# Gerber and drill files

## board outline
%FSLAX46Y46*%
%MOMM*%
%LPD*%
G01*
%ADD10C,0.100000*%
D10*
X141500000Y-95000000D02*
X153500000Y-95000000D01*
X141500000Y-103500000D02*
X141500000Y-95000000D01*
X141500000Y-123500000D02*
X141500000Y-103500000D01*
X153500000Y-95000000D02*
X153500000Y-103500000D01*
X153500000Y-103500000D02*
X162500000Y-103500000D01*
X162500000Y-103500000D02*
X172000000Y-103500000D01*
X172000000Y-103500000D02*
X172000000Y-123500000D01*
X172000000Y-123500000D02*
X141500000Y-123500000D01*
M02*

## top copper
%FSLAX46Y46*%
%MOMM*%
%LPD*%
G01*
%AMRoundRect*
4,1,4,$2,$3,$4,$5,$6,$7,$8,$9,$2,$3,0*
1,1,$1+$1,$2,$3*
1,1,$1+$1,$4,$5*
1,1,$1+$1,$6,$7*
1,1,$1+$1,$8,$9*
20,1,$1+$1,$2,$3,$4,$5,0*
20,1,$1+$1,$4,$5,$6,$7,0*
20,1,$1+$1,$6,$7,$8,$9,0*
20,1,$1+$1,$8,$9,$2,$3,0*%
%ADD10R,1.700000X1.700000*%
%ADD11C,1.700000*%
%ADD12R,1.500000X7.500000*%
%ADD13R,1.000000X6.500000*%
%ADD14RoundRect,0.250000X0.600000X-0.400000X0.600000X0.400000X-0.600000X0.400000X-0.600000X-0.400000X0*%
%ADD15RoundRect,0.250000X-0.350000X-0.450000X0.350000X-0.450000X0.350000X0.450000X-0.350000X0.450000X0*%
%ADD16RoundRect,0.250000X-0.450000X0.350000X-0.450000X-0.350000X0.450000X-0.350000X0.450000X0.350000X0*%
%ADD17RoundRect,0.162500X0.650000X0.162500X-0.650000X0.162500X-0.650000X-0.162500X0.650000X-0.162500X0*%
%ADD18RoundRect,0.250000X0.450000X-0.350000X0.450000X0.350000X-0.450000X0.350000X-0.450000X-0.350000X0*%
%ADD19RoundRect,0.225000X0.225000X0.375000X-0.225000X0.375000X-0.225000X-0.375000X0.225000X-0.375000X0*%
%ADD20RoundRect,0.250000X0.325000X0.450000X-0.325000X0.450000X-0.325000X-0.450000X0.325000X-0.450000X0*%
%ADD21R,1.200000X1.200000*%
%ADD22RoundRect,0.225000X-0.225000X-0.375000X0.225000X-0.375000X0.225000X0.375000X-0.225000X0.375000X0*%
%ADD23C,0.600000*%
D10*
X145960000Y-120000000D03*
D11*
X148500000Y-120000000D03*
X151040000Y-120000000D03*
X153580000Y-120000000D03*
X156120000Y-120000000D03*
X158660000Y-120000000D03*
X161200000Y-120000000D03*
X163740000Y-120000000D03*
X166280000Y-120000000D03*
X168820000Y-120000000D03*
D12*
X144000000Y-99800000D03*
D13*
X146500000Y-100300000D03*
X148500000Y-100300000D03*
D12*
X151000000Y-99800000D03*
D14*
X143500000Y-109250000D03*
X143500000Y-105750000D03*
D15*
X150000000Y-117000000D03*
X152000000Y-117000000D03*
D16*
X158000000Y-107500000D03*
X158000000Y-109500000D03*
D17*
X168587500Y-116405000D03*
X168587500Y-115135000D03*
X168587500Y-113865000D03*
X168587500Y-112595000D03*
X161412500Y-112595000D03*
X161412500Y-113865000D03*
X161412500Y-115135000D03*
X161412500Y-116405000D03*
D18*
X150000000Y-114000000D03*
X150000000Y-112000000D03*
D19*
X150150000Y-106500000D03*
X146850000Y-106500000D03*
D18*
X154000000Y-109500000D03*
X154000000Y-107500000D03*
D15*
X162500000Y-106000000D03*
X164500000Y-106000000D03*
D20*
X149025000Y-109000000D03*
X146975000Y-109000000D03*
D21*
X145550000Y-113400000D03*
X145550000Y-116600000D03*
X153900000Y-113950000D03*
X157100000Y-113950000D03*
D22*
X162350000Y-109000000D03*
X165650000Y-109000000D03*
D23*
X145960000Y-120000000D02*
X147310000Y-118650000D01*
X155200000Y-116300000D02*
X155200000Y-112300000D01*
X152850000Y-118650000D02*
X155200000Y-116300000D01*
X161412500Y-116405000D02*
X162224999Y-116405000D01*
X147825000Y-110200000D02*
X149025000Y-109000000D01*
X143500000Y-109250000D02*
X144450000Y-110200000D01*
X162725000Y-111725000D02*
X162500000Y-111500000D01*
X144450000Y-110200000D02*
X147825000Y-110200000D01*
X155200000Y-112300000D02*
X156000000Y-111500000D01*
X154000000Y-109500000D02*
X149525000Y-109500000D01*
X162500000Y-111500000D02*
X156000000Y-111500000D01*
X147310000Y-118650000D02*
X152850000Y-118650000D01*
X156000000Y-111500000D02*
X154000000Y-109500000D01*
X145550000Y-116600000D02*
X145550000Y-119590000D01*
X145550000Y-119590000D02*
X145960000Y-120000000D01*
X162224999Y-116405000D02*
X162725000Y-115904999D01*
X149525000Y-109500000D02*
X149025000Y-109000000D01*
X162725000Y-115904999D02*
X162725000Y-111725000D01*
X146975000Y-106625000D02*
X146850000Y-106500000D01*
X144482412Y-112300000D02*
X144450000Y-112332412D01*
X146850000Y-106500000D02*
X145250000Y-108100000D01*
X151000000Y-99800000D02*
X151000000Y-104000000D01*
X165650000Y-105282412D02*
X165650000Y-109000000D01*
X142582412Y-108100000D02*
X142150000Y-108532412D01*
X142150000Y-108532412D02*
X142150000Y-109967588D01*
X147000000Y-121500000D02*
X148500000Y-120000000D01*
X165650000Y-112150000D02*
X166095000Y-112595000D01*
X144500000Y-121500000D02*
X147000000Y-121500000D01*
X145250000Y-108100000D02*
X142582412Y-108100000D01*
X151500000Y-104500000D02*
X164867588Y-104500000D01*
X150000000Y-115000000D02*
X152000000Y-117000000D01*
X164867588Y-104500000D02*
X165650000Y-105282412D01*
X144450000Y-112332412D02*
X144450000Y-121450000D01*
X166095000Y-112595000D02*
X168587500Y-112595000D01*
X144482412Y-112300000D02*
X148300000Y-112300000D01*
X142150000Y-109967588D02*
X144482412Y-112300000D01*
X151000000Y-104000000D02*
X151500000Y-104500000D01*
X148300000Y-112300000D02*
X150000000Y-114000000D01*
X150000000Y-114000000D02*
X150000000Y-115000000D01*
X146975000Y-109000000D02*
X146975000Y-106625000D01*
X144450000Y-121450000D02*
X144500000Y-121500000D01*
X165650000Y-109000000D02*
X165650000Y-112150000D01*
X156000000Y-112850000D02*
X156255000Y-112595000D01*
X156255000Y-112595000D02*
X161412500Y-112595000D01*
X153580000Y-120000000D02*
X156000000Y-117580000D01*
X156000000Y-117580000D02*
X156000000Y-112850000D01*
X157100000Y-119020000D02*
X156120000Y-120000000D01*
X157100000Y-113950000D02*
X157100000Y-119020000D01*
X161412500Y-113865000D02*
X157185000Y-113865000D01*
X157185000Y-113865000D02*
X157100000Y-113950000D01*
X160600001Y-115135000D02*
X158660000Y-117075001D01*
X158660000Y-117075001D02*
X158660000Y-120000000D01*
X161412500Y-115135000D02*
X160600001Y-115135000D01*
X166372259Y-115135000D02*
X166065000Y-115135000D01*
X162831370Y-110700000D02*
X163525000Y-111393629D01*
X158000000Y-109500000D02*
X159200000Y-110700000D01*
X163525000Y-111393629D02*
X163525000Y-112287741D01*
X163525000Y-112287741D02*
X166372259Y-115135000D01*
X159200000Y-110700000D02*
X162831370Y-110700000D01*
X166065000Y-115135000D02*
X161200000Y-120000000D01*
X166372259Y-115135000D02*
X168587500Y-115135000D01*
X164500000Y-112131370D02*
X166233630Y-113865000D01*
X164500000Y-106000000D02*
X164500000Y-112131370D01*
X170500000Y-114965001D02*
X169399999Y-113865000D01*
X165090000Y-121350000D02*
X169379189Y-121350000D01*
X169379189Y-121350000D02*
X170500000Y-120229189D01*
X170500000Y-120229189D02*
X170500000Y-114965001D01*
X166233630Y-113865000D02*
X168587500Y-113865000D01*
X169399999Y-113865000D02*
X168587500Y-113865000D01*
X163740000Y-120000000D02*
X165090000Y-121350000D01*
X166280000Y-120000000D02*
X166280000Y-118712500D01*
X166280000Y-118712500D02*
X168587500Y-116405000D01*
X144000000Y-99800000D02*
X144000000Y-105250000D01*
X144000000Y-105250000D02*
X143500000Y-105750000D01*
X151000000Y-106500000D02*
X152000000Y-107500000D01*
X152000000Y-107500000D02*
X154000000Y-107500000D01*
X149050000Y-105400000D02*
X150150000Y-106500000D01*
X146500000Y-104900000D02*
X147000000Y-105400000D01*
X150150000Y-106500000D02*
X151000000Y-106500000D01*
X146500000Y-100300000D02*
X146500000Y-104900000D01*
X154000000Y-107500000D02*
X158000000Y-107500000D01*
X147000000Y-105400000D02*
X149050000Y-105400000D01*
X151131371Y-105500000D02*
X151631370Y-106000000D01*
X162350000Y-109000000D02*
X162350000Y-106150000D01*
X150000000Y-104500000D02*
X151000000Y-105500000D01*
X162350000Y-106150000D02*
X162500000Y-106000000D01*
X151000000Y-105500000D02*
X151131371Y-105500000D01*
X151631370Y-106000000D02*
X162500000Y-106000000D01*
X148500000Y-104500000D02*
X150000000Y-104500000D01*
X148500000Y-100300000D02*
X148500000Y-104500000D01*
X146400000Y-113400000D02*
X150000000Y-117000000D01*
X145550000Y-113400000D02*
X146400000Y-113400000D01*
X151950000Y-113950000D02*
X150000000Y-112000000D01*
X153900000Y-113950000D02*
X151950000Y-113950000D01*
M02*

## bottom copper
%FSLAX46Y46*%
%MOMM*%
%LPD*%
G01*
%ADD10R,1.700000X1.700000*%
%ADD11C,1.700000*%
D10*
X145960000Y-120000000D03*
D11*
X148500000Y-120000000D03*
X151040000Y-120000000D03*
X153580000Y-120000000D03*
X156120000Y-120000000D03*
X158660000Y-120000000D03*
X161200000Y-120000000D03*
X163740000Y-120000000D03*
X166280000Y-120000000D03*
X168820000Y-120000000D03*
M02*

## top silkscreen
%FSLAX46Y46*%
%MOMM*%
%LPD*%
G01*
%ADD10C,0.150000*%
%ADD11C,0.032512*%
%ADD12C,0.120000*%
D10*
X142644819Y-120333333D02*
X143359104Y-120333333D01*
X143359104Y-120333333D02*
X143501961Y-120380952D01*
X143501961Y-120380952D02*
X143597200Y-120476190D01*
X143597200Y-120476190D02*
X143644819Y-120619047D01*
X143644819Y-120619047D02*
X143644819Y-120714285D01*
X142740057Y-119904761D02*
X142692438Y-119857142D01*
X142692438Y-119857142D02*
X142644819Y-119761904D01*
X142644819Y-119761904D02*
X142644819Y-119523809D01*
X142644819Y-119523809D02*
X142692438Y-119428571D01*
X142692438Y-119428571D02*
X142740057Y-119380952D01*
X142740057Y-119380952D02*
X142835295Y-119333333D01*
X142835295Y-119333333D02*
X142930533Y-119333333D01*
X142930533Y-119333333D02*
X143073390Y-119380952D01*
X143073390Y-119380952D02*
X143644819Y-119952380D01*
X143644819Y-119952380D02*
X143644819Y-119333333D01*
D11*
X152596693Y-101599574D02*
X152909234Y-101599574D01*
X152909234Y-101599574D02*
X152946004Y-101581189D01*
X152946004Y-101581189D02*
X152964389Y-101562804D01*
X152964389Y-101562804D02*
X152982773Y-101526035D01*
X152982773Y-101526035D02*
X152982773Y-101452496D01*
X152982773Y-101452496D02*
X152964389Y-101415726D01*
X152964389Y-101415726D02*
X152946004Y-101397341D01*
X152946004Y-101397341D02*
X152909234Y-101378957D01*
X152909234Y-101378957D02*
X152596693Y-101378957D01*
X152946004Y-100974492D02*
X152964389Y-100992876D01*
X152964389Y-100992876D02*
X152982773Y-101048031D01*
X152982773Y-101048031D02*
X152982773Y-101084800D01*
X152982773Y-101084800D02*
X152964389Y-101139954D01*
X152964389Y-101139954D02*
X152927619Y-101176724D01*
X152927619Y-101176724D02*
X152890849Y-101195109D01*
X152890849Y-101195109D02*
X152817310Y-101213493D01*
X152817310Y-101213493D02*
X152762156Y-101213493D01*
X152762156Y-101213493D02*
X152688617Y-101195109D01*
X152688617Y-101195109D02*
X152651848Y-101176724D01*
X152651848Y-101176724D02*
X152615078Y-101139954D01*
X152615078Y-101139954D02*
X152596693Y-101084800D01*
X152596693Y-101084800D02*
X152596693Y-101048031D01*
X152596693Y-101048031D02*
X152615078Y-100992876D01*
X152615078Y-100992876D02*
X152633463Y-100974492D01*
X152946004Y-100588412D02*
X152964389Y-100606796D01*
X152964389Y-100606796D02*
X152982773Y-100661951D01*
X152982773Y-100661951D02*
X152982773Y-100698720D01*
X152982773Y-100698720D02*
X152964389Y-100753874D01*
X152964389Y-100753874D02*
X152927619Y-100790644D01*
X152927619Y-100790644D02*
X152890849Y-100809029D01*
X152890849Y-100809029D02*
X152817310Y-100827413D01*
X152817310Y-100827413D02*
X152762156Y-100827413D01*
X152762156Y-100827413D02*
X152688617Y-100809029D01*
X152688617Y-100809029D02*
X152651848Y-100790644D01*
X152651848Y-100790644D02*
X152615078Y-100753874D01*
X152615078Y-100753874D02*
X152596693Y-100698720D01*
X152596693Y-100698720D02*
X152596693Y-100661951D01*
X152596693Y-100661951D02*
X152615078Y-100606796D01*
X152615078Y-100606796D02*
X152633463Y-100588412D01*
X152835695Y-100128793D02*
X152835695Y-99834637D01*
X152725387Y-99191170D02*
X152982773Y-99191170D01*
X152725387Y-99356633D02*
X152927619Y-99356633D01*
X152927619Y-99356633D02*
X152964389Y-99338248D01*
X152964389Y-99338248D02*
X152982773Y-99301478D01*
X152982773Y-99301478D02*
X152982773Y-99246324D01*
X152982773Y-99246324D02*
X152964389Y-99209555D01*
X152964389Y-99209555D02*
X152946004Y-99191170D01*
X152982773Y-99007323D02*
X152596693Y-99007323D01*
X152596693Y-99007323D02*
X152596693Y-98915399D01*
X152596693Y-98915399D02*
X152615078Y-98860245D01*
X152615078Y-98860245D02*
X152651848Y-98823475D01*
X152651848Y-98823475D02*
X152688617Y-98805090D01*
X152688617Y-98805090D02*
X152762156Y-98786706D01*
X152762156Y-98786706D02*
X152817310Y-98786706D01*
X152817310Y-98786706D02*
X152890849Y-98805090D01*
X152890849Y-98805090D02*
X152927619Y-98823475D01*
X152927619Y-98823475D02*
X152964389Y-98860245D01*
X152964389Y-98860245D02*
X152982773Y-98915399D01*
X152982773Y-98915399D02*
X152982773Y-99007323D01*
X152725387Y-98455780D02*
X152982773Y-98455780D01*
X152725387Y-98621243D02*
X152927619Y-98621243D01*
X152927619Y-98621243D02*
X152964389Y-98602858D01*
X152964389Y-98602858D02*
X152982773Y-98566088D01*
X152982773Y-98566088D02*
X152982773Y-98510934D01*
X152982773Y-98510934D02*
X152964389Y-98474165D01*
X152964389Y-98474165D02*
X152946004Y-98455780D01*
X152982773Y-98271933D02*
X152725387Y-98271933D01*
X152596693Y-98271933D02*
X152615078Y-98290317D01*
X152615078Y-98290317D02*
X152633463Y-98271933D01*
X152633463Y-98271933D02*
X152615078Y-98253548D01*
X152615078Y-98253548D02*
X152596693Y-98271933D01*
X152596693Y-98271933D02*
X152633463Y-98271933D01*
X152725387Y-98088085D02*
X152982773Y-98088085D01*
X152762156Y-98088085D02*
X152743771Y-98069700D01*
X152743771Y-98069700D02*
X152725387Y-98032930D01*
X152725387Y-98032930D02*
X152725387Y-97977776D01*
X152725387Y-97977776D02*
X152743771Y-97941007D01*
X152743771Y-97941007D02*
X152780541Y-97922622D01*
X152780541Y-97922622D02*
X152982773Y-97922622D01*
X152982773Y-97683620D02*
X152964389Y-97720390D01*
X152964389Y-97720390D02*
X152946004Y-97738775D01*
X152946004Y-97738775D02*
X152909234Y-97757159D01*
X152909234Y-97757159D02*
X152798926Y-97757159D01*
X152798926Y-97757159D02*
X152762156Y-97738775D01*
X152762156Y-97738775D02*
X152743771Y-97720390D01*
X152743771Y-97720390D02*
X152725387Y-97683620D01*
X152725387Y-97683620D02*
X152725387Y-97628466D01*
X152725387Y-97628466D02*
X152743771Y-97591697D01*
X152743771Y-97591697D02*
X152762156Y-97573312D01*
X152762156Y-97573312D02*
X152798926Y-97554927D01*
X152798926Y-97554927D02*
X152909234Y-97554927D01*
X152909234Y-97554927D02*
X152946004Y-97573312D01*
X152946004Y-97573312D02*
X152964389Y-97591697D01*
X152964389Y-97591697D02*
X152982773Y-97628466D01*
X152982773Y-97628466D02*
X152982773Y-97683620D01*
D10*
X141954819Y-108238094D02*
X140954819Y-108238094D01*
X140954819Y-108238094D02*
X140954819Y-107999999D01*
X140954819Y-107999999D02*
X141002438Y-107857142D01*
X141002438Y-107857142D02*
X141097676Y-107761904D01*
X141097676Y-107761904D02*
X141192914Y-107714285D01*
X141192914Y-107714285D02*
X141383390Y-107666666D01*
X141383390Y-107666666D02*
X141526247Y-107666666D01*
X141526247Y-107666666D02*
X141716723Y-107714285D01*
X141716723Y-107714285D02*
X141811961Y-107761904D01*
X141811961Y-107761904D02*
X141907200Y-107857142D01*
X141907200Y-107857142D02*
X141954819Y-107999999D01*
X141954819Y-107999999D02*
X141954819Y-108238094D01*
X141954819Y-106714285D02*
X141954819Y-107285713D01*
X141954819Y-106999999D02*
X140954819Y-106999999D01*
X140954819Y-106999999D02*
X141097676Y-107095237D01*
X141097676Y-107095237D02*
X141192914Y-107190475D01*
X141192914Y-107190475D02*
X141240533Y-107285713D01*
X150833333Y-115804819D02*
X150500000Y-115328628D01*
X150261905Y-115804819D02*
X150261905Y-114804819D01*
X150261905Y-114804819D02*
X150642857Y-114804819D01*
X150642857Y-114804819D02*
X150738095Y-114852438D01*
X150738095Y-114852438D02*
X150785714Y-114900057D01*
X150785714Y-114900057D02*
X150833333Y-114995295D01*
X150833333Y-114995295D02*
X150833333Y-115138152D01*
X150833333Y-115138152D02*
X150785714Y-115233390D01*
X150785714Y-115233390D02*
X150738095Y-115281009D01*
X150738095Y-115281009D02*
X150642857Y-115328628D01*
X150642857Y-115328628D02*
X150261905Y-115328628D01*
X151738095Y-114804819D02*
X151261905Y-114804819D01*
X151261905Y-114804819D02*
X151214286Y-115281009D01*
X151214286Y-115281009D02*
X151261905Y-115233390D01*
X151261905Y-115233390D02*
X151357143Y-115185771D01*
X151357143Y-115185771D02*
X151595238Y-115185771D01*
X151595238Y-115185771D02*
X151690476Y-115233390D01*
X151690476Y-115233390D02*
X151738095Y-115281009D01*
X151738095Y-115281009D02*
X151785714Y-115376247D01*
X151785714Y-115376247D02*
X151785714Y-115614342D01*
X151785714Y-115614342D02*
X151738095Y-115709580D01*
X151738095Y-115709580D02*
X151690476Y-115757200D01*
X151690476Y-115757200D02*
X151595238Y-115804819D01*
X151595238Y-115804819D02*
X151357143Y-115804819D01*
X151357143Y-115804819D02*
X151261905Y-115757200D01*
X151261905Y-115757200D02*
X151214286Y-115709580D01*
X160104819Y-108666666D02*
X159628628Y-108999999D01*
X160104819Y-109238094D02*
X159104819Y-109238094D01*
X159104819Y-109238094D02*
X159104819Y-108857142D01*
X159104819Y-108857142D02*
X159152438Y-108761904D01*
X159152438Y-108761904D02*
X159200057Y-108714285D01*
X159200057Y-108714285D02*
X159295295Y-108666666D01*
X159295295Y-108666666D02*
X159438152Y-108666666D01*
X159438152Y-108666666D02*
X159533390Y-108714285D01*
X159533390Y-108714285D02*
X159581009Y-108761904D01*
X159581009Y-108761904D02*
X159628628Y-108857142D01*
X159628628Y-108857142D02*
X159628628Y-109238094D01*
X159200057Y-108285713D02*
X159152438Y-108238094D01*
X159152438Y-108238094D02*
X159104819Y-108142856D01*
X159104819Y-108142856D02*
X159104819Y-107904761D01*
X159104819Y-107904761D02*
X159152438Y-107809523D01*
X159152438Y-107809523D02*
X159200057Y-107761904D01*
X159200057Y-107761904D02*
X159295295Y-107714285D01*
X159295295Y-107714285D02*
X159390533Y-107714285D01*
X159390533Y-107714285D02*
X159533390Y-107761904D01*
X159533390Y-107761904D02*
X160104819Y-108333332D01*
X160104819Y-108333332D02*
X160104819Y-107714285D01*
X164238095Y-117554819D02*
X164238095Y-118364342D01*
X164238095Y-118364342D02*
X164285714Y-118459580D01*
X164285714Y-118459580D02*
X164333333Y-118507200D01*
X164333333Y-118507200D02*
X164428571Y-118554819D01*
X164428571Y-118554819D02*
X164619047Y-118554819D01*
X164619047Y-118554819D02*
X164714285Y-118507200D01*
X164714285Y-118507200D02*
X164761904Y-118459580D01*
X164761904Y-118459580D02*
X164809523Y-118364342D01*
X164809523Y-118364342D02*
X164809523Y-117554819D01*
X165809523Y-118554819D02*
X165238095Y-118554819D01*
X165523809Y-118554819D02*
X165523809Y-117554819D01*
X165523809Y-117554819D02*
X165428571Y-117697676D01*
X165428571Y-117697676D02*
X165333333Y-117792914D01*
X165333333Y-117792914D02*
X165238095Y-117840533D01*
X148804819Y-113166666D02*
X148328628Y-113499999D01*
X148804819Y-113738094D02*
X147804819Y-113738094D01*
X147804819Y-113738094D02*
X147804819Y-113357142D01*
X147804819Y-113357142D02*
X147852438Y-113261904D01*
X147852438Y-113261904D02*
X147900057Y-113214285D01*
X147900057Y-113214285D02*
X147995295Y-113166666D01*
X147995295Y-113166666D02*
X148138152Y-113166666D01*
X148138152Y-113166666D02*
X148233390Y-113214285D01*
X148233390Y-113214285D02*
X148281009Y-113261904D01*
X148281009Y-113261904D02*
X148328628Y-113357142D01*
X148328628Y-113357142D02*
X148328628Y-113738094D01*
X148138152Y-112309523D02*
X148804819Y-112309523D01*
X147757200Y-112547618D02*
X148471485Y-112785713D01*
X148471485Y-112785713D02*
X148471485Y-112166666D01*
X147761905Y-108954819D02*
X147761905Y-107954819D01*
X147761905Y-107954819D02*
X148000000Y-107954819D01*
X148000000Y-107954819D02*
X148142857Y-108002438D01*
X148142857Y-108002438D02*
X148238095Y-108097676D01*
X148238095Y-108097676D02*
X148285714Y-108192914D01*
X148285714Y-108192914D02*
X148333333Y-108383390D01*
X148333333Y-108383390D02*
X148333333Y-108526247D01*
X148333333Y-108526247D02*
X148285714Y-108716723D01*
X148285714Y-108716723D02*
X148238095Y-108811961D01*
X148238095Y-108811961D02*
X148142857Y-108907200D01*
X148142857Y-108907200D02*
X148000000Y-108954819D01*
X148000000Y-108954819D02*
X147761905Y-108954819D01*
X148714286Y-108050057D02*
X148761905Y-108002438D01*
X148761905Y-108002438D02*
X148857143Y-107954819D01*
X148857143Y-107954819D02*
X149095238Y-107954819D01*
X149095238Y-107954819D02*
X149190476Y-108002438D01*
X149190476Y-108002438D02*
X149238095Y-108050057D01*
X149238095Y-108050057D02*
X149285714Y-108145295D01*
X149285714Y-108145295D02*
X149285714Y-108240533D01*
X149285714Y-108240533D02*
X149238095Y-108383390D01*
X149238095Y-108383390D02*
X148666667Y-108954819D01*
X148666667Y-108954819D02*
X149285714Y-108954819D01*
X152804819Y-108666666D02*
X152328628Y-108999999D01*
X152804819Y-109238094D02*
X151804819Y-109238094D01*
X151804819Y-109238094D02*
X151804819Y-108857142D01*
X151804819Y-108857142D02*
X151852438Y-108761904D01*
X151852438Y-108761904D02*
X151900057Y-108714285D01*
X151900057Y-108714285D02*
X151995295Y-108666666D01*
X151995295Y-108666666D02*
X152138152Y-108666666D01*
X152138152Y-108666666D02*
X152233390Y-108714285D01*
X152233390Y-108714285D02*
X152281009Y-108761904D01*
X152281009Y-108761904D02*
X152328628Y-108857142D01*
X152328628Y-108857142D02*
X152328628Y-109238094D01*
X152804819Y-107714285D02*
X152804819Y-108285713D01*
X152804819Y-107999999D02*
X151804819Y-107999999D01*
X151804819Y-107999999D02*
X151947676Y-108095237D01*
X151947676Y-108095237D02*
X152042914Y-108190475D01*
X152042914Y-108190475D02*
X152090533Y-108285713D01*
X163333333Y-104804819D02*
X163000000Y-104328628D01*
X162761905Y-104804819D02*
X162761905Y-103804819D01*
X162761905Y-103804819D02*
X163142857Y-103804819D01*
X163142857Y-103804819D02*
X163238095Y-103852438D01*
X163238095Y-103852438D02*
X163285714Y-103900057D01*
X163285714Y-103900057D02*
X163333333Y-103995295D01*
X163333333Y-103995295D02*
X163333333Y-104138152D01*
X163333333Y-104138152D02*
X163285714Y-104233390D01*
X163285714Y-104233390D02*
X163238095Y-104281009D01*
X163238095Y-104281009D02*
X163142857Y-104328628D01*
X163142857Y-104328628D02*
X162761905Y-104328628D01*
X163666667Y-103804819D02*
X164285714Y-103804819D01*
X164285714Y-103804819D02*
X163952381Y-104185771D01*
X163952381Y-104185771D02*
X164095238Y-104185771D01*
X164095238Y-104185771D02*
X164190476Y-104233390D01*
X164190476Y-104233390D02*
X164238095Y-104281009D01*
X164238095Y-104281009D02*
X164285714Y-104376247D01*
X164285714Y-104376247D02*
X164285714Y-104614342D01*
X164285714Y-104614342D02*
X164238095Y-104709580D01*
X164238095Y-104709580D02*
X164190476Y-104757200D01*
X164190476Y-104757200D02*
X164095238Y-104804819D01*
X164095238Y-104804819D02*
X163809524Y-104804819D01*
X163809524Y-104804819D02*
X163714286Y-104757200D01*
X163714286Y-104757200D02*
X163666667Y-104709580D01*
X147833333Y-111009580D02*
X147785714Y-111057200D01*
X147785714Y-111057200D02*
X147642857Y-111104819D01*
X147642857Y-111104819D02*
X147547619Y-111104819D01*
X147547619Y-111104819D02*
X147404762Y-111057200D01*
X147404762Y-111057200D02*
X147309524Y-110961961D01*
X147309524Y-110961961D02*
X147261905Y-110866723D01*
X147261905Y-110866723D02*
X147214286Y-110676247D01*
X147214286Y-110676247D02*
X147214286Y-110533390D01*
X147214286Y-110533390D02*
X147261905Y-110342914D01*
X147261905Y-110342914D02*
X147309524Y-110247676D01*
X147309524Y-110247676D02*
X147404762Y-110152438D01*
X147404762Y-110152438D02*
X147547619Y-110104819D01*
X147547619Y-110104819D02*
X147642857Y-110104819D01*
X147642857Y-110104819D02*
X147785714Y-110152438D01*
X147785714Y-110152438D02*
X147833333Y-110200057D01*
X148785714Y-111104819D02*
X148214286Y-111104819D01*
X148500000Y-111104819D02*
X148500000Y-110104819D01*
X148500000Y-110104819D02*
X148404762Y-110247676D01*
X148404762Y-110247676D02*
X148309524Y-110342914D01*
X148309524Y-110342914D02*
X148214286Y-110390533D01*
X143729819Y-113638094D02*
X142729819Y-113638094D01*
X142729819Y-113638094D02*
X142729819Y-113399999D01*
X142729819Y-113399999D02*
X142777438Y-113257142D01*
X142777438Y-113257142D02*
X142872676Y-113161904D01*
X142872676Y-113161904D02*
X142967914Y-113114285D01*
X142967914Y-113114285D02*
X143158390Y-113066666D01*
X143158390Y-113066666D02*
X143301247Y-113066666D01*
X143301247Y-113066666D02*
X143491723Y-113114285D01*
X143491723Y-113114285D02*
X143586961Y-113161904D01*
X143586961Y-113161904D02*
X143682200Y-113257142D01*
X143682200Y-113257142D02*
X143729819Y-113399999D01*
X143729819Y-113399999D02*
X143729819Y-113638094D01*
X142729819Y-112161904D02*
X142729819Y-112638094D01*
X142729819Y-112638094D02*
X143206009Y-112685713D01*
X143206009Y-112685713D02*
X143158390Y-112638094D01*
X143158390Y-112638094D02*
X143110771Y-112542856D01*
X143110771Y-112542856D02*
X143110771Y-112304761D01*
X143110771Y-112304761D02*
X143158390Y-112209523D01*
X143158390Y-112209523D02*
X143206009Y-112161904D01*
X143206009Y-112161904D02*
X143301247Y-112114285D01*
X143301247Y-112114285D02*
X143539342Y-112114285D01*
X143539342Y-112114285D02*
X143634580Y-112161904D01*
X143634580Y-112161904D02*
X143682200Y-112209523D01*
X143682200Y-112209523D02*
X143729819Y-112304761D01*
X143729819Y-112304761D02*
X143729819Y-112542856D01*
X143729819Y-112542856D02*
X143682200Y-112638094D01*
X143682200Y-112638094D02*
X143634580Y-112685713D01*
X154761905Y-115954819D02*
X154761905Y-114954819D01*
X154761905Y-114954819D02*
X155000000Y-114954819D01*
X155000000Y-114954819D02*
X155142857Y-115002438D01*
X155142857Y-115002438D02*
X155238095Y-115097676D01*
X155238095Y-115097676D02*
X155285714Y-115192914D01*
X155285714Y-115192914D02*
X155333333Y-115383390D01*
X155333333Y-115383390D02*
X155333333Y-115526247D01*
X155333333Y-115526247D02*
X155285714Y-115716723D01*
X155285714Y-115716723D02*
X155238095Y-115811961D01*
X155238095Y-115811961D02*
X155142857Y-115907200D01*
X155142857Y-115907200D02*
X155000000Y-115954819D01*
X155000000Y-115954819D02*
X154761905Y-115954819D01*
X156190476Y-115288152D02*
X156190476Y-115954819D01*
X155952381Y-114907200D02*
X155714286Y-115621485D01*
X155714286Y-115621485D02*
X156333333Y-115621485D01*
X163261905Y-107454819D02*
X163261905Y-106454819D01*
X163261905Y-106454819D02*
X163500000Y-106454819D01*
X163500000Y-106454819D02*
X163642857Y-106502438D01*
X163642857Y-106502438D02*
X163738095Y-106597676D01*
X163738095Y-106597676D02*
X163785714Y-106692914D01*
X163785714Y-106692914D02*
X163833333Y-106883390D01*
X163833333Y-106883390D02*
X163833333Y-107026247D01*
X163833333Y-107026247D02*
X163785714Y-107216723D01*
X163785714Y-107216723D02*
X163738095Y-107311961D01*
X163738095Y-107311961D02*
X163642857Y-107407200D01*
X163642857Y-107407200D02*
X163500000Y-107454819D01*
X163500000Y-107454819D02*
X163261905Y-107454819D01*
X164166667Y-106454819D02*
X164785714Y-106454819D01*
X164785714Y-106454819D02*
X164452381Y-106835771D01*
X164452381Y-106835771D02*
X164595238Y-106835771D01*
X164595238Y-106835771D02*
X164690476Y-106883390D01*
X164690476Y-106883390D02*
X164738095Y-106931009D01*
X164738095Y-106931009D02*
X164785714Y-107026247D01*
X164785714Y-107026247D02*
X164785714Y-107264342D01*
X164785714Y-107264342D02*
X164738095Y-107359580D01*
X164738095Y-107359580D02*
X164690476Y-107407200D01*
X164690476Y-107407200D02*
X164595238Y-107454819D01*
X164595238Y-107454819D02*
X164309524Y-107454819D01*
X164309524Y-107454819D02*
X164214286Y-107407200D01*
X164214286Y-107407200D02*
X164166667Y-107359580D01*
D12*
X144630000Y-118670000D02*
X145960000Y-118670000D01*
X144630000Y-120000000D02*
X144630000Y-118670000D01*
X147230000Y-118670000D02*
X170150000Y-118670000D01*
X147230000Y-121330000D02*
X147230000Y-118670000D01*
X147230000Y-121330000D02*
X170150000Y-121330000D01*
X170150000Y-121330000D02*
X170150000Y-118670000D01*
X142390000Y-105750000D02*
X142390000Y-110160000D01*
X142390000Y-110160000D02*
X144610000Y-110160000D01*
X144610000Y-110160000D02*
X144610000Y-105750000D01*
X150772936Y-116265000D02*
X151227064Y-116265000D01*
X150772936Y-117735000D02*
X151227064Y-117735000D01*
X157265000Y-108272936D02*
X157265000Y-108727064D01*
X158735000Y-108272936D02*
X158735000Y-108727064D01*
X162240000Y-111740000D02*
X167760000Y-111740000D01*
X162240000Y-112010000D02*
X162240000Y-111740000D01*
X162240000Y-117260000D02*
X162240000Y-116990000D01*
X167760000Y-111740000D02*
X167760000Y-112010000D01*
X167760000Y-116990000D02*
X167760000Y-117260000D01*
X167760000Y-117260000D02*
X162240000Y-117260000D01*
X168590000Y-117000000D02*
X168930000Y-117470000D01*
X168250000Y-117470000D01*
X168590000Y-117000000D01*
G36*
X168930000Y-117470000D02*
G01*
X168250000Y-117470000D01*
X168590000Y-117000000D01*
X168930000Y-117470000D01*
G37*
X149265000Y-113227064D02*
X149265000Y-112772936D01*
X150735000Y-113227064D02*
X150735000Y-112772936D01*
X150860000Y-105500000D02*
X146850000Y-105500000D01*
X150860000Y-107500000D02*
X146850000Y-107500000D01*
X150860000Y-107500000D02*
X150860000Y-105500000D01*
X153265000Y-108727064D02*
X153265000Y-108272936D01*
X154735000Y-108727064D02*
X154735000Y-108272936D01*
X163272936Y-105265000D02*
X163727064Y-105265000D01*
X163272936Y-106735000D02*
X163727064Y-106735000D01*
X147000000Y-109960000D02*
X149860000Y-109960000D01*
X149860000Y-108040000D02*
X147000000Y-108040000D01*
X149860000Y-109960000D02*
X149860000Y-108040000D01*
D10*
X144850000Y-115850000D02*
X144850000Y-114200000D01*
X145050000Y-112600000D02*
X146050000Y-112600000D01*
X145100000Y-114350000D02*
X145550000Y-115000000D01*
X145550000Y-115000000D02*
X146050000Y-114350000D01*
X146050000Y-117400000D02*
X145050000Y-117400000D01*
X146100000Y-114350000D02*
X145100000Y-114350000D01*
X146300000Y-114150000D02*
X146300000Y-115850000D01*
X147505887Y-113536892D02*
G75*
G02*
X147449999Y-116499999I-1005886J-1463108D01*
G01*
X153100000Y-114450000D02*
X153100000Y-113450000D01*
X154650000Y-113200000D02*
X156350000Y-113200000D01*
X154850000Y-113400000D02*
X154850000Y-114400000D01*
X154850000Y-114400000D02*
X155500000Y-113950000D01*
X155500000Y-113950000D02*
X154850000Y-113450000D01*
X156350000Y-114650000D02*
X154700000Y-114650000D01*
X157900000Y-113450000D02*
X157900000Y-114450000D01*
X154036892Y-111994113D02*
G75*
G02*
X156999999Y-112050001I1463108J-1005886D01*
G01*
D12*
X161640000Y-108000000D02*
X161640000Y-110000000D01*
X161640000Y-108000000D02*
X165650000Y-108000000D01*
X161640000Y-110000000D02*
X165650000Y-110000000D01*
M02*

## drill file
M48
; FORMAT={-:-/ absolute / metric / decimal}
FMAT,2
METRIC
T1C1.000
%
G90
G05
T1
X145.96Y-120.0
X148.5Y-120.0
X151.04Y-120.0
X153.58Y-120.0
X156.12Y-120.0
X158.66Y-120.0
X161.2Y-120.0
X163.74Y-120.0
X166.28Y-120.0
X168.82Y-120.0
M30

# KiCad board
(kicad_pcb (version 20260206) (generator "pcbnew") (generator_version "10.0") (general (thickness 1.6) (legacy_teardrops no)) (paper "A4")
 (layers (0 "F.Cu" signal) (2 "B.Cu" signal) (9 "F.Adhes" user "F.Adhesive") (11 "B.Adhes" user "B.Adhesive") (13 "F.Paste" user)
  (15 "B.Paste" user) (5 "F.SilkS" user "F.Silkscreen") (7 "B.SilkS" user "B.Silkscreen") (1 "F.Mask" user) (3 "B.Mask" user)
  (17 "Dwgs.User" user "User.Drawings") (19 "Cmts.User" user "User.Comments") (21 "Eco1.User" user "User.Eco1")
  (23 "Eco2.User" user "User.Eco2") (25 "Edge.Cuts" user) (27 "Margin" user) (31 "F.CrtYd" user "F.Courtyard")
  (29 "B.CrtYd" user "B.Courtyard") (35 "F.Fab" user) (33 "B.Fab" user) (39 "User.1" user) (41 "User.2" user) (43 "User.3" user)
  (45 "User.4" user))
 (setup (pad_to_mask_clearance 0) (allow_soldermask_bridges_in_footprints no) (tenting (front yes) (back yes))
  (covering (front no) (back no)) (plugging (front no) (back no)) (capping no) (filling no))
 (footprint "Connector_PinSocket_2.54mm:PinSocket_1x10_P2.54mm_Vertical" (layer "F.Cu") (at 145.96 120 90)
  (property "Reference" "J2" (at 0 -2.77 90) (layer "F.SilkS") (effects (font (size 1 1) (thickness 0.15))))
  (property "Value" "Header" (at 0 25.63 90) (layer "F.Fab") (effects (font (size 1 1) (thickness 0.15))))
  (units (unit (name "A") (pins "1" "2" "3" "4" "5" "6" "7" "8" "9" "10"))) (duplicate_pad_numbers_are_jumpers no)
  (fp_line (start 1.33 -1.33) (end 1.33 0) (stroke (width 0.12) (type solid)) (layer "F.SilkS"))
  (fp_line (start 0 -1.33) (end 1.33 -1.33) (stroke (width 0.12) (type solid)) (layer "F.SilkS"))
  (fp_line (start 1.33 1.27) (end 1.33 24.19) (stroke (width 0.12) (type solid)) (layer "F.SilkS"))
  (fp_line (start -1.33 1.27) (end 1.33 1.27) (stroke (width 0.12) (type solid)) (layer "F.SilkS"))
  (fp_line (start -1.33 1.27) (end -1.33 24.19) (stroke (width 0.12) (type solid)) (layer "F.SilkS"))
  (fp_line (start -1.33 24.19) (end 1.33 24.19) (stroke (width 0.12) (type solid)) (layer "F.SilkS"))
  (pad "1" thru_hole rect (at 0 0 90) (size 1.7 1.7) (drill 1) (layers "*.Cu" "*.Mask") (remove_unused_layers no) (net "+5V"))
  (pad "2" thru_hole circle (at 0 2.54 90) (size 1.7 1.7) (drill 1) (layers "*.Cu" "*.Mask") (remove_unused_layers no) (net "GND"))
  (pad "3" thru_hole circle (at 0 5.08 90) (size 1.7 1.7) (drill 1) (layers "*.Cu" "*.Mask") (remove_unused_layers no)
   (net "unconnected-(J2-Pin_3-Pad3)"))
  (pad "4" thru_hole circle (at 0 7.62 90) (size 1.7 1.7) (drill 1) (layers "*.Cu" "*.Mask") (remove_unused_layers no)
   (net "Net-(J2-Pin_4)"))
  (pad "5" thru_hole circle (at 0 10.16 90) (size 1.7 1.7) (drill 1) (layers "*.Cu" "*.Mask") (remove_unused_layers no) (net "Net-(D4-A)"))
  (pad "6" thru_hole circle (at 0 12.7 90) (size 1.7 1.7) (drill 1) (layers "*.Cu" "*.Mask") (remove_unused_layers no)
   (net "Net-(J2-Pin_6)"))
  (pad "7" thru_hole circle (at 0 15.24 90) (size 1.7 1.7) (drill 1) (layers "*.Cu" "*.Mask") (remove_unused_layers no)
   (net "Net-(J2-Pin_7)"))
  (pad "8" thru_hole circle (at 0 17.78 90) (size 1.7 1.7) (drill 1) (layers "*.Cu" "*.Mask") (remove_unused_layers no)
   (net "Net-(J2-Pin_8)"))
  (pad "9" thru_hole circle (at 0 20.32 90) (size 1.7 1.7) (drill 1) (layers "*.Cu" "*.Mask") (remove_unused_layers no)
   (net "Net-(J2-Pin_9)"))
  (pad "10" thru_hole circle (at 0 22.86 90) (size 1.7 1.7) (drill 1) (layers "*.Cu" "*.Mask") (remove_unused_layers no)
   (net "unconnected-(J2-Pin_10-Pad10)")))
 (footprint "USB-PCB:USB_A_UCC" (layer "F.Cu") (at 147.5 100 -90)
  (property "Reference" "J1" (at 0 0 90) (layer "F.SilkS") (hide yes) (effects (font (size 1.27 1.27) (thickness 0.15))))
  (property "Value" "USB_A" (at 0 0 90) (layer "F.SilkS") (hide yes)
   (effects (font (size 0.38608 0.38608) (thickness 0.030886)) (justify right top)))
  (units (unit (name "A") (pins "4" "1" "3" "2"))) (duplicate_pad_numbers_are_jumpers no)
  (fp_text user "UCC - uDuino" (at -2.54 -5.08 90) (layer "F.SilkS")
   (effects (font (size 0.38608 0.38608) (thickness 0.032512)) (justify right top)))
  (pad "1" smd rect (at -0.2 3.5 270) (size 7.5 1.5) (layers "F.Cu" "F.Mask" "F.Paste") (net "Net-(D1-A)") (solder_mask_margin 0.1016))
  (pad "2" smd rect (at 0.3 1 270) (size 6.5 1) (layers "F.Cu" "F.Mask" "F.Paste") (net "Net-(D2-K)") (solder_mask_margin 0.1016))
  (pad "3" smd rect (at 0.3 -1 270) (size 6.5 1) (layers "F.Cu" "F.Mask" "F.Paste") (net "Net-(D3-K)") (solder_mask_margin 0.1016))
  (pad "4" smd rect (at -0.2 -3.5 270) (size 7.5 1.5) (layers "F.Cu" "F.Mask" "F.Paste") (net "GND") (solder_mask_margin 0.1016)))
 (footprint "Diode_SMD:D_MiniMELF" (layer "F.Cu") (at 143.5 107.5 90)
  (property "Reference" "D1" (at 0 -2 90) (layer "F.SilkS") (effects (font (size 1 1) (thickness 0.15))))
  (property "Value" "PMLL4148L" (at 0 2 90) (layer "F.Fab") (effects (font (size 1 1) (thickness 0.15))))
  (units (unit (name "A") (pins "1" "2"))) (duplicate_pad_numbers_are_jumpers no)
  (fp_line (start 1.75 -1.11) (end -2.66 -1.11) (stroke (width 0.12) (type solid)) (layer "F.SilkS"))
  (fp_line (start -2.66 -1.11) (end -2.66 1.11) (stroke (width 0.12) (type solid)) (layer "F.SilkS"))
  (fp_line (start -2.66 1.11) (end 1.75 1.11) (stroke (width 0.12) (type solid)) (layer "F.SilkS"))
  (pad "1" smd roundrect (at -1.75 0 90) (size 1.3 1.7) (layers "F.Cu" "F.Mask" "F.Paste") (roundrect_rratio 0.1923076923) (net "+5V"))
  (pad "2" smd roundrect (at 1.75 0 90) (size 1.3 1.7) (layers "F.Cu" "F.Mask" "F.Paste") (roundrect_rratio 0.1923076923) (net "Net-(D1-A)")))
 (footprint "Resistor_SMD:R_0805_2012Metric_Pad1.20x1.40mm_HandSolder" (layer "F.Cu") (at 151 117)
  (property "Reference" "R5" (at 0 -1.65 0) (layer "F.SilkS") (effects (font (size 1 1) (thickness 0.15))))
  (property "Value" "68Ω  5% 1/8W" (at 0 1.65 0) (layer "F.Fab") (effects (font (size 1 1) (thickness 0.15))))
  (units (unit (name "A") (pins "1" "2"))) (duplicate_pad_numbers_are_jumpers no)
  (fp_line (start -0.227064 -0.735) (end 0.227064 -0.735) (stroke (width 0.12) (type solid)) (layer "F.SilkS"))
  (fp_line (start -0.227064 0.735) (end 0.227064 0.735) (stroke (width 0.12) (type solid)) (layer "F.SilkS"))
  (pad "1" smd roundrect (at -1 0) (size 1.2 1.4) (layers "F.Cu" "F.Mask" "F.Paste") (roundrect_rratio 0.208333) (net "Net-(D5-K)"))
  (pad "2" smd roundrect (at 1 0) (size 1.2 1.4) (layers "F.Cu" "F.Mask" "F.Paste") (roundrect_rratio 0.208333) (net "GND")))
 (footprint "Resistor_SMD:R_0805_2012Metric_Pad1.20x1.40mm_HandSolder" (layer "F.Cu") (at 158 108.5 -90)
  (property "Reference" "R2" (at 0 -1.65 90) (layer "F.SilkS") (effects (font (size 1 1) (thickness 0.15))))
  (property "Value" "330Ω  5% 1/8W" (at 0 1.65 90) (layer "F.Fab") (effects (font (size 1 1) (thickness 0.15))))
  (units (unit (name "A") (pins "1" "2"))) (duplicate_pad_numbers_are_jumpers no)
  (fp_line (start -0.227064 0.735) (end 0.227064 0.735) (stroke (width 0.12) (type solid)) (layer "F.SilkS"))
  (fp_line (start -0.227064 -0.735) (end 0.227064 -0.735) (stroke (width 0.12) (type solid)) (layer "F.SilkS"))
  (pad "1" smd roundrect (at -1 0 270) (size 1.2 1.4) (layers "F.Cu" "F.Mask" "F.Paste") (roundrect_rratio 0.208333) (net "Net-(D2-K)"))
  (pad "2" smd roundrect (at 1 0 270) (size 1.2 1.4) (layers "F.Cu" "F.Mask" "F.Paste") (roundrect_rratio 0.208333) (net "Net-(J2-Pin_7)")))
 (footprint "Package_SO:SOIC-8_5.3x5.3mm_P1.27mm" (layer "F.Cu") (at 165 114.5 180)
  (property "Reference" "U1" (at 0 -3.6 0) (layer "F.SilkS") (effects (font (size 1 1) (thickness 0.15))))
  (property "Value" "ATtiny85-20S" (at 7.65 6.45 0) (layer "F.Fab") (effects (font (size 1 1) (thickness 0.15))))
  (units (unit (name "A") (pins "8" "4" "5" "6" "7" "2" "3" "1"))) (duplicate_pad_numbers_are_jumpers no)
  (fp_line (start 2.76 2.76) (end -2.76 2.76) (stroke (width 0.12) (type solid)) (layer "F.SilkS"))
  (fp_line (start 2.76 2.49) (end 2.76 2.76) (stroke (width 0.12) (type solid)) (layer "F.SilkS"))
  (fp_line (start 2.76 -2.76) (end 2.76 -2.49) (stroke (width 0.12) (type solid)) (layer "F.SilkS"))
  (fp_line (start -2.76 2.76) (end -2.76 2.49) (stroke (width 0.12) (type solid)) (layer "F.SilkS"))
  (fp_line (start -2.76 -2.49) (end -2.76 -2.76) (stroke (width 0.12) (type solid)) (layer "F.SilkS"))
  (fp_line (start -2.76 -2.76) (end 2.76 -2.76) (stroke (width 0.12) (type solid)) (layer "F.SilkS"))
  (fp_poly (pts (xy -3.59 -2.5) (xy -3.93 -2.97) (xy -3.25 -2.97)) (stroke (width 0.12) (type solid)) (fill yes) (layer "F.SilkS"))
  (pad "1" smd roundrect (at -3.5875 -1.905 180) (size 1.625 0.65) (layers "F.Cu" "F.Mask" "F.Paste") (roundrect_rratio 0.25)
   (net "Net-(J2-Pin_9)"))
  (pad "2" smd roundrect (at -3.5875 -0.635 180) (size 1.625 0.65) (layers "F.Cu" "F.Mask" "F.Paste") (roundrect_rratio 0.25)
   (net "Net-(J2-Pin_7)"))
  (pad "3" smd roundrect (at -3.5875 0.635 180) (size 1.625 0.65) (layers "F.Cu" "F.Mask" "F.Paste") (roundrect_rratio 0.25)
   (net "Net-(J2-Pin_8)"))
  (pad "4" smd roundrect (at -3.5875 1.905 180) (size 1.625 0.65) (layers "F.Cu" "F.Mask" "F.Paste") (roundrect_rratio 0.25) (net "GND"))
  (pad "5" smd roundrect (at 3.5875 1.905 180) (size 1.625 0.65) (layers "F.Cu" "F.Mask" "F.Paste") (roundrect_rratio 0.25)
   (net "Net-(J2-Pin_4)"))
  (pad "6" smd roundrect (at 3.5875 0.635 180) (size 1.625 0.65) (layers "F.Cu" "F.Mask" "F.Paste") (roundrect_rratio 0.25)
   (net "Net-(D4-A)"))
  (pad "7" smd roundrect (at 3.5875 -0.635 180) (size 1.625 0.65) (layers "F.Cu" "F.Mask" "F.Paste") (roundrect_rratio 0.25)
   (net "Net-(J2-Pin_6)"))
  (pad "8" smd roundrect (at 3.5875 -1.905 180) (size 1.625 0.65) (layers "F.Cu" "F.Mask" "F.Paste") (roundrect_rratio 0.25) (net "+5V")))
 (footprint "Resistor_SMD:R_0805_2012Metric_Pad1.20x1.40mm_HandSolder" (layer "F.Cu") (at 150 113 90)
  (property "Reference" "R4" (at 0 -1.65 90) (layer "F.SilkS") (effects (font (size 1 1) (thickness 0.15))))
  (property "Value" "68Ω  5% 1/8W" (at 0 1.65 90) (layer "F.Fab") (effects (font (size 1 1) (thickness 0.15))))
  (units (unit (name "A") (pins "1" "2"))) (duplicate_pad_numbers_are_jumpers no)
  (fp_line (start -0.227064 -0.735) (end 0.227064 -0.735) (stroke (width 0.12) (type solid)) (layer "F.SilkS"))
  (fp_line (start -0.227064 0.735) (end 0.227064 0.735) (stroke (width 0.12) (type solid)) (layer "F.SilkS"))
  (pad "1" smd roundrect (at -1 0 90) (size 1.2 1.4) (layers "F.Cu" "F.Mask" "F.Paste") (roundrect_rratio 0.208333) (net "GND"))
  (pad "2" smd roundrect (at 1 0 90) (size 1.2 1.4) (layers "F.Cu" "F.Mask" "F.Paste") (roundrect_rratio 0.208333) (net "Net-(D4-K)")))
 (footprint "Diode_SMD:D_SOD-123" (layer "F.Cu") (at 148.5 106.5 180)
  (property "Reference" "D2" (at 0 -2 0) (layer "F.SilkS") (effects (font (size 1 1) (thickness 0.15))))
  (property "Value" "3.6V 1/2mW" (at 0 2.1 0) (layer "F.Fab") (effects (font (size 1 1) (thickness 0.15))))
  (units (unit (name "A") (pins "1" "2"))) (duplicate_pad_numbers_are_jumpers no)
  (fp_line (start -2.36 1) (end 1.65 1) (stroke (width 0.12) (type solid)) (layer "F.SilkS"))
  (fp_line (start -2.36 -1) (end 1.65 -1) (stroke (width 0.12) (type solid)) (layer "F.SilkS"))
  (fp_line (start -2.36 -1) (end -2.36 1) (stroke (width 0.12) (type solid)) (layer "F.SilkS"))
  (pad "1" smd roundrect (at -1.65 0 180) (size 0.9 1.2) (layers "F.Cu" "F.Mask" "F.Paste") (roundrect_rratio 0.25) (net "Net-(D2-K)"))
  (pad "2" smd roundrect (at 1.65 0 180) (size 0.9 1.2) (layers "F.Cu" "F.Mask" "F.Paste") (roundrect_rratio 0.25) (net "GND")))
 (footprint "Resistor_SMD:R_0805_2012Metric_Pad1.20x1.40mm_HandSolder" (layer "F.Cu") (at 154 108.5 90)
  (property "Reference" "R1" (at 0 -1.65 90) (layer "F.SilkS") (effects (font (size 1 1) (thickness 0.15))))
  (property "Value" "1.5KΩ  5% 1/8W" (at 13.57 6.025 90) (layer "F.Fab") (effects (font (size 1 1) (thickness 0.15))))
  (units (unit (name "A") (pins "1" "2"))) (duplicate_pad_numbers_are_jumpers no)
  (fp_line (start -0.227064 -0.735) (end 0.227064 -0.735) (stroke (width 0.12) (type solid)) (layer "F.SilkS"))
  (fp_line (start -0.227064 0.735) (end 0.227064 0.735) (stroke (width 0.12) (type solid)) (layer "F.SilkS"))
  (pad "1" smd roundrect (at -1 0 90) (size 1.2 1.4) (layers "F.Cu" "F.Mask" "F.Paste") (roundrect_rratio 0.208333) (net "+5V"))
  (pad "2" smd roundrect (at 1 0 90) (size 1.2 1.4) (layers "F.Cu" "F.Mask" "F.Paste") (roundrect_rratio 0.208333) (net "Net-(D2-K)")))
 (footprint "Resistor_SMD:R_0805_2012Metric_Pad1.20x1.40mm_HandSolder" (layer "F.Cu") (at 163.5 106)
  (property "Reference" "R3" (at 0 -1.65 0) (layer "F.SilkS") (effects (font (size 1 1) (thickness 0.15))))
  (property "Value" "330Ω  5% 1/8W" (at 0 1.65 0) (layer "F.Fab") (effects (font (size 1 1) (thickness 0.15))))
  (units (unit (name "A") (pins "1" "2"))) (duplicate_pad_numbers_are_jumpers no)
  (fp_line (start -0.227064 -0.735) (end 0.227064 -0.735) (stroke (width 0.12) (type solid)) (layer "F.SilkS"))
  (fp_line (start -0.227064 0.735) (end 0.227064 0.735) (stroke (width 0.12) (type solid)) (layer "F.SilkS"))
  (pad "1" smd roundrect (at -1 0) (size 1.2 1.4) (layers "F.Cu" "F.Mask" "F.Paste") (roundrect_rratio 0.208333) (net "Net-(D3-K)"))
  (pad "2" smd roundrect (at 1 0) (size 1.2 1.4) (layers "F.Cu" "F.Mask" "F.Paste") (roundrect_rratio 0.208333) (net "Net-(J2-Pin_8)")))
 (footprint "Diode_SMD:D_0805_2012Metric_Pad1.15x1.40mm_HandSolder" (layer "F.Cu") (at 148 109 180)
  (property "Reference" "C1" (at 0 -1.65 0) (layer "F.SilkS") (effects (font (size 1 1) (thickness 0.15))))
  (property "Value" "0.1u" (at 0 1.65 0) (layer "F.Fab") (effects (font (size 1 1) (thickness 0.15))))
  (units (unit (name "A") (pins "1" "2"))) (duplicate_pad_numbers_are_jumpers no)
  (fp_line (start 1 -0.96) (end -1.86 -0.96) (stroke (width 0.12) (type solid)) (layer "F.SilkS"))
  (fp_line (start -1.86 0.96) (end 1 0.96) (stroke (width 0.12) (type solid)) (layer "F.SilkS"))
  (fp_line (start -1.86 -0.96) (end -1.86 0.96) (stroke (width 0.12) (type solid)) (layer "F.SilkS"))
  (pad "1" smd roundrect (at -1.025 0 180) (size 1.15 1.4) (layers "F.Cu" "F.Mask" "F.Paste") (roundrect_rratio 0.217391) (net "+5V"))
  (pad "2" smd roundrect (at 1.025 0 180) (size 1.15 1.4) (layers "F.Cu" "F.Mask" "F.Paste") (roundrect_rratio 0.217391) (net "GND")))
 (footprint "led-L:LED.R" (layer "F.Cu") (at 146 115.5 -90)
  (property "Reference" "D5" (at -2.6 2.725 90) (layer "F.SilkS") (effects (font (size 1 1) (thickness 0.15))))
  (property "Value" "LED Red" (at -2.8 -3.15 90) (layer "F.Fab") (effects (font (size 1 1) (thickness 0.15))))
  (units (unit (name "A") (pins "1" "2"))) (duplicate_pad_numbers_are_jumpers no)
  (fp_line (start 0.35 1.15) (end -1.3 1.15) (stroke (width 0.15) (type solid)) (layer "F.SilkS"))
  (fp_line (start -2.9 0.95) (end -2.9 -0.05) (stroke (width 0.15) (type solid)) (layer "F.SilkS"))
  (fp_line (start -1.15 0.9) (end -0.5 0.45) (stroke (width 0.15) (type solid)) (layer "F.SilkS"))
  (fp_line (start -0.5 0.45) (end -1.15 -0.05) (stroke (width 0.15) (type solid)) (layer "F.SilkS"))
  (fp_line (start 1.9 -0.05) (end 1.9 0.95) (stroke (width 0.15) (type solid)) (layer "F.SilkS"))
  (fp_line (start -1.15 -0.1) (end -1.15 0.9) (stroke (width 0.15) (type solid)) (layer "F.SilkS"))
  (fp_line (start -1.35 -0.3) (end 0.35 -0.3) (stroke (width 0.15) (type solid)) (layer "F.SilkS"))
  (fp_arc (start -1.963108 -1.505887) (mid -0.466517 -2.275211) (end 0.999999 -1.449999) (stroke (width 0.15) (type solid))
   (layer "F.SilkS"))
  (pad "1" smd rect (at -2.1 0.45 270) (size 1.2 1.2) (layers "F.Cu" "F.Mask" "F.Paste") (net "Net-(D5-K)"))
  (pad "2" smd rect (at 1.1 0.45 270) (size 1.2 1.2) (layers "F.Cu" "F.Mask" "F.Paste") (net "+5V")))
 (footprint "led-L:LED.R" (layer "F.Cu") (at 156 113.5)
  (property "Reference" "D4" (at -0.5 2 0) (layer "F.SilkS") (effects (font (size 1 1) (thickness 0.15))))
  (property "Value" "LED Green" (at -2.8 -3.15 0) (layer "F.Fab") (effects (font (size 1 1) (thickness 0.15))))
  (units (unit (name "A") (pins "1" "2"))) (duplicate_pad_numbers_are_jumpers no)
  (fp_line (start -2.9 0.95) (end -2.9 -0.05) (stroke (width 0.15) (type solid)) (layer "F.SilkS"))
  (fp_line (start -1.35 -0.3) (end 0.35 -0.3) (stroke (width 0.15) (type solid)) (layer "F.SilkS"))
  (fp_line (start -1.15 -0.1) (end -1.15 0.9) (stroke (width 0.15) (type solid)) (layer "F.SilkS"))
  (fp_line (start -1.15 0.9) (end -0.5 0.45) (stroke (width 0.15) (type solid)) (layer "F.SilkS"))
  (fp_line (start -0.5 0.45) (end -1.15 -0.05) (stroke (width 0.15) (type solid)) (layer "F.SilkS"))
  (fp_line (start 0.35 1.15) (end -1.3 1.15) (stroke (width 0.15) (type solid)) (layer "F.SilkS"))
  (fp_line (start 1.9 -0.05) (end 1.9 0.95) (stroke (width 0.15) (type solid)) (layer "F.SilkS"))
  (fp_arc (start -1.963108 -1.505887) (mid -0.466517 -2.275211) (end 0.999999 -1.449999) (stroke (width 0.15) (type solid))
   (layer "F.SilkS"))
  (pad "1" smd rect (at -2.1 0.45) (size 1.2 1.2) (layers "F.Cu" "F.Mask" "F.Paste") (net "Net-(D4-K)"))
  (pad "2" smd rect (at 1.1 0.45) (size 1.2 1.2) (layers "F.Cu" "F.Mask" "F.Paste") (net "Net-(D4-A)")))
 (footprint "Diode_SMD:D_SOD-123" (layer "F.Cu") (at 164 109)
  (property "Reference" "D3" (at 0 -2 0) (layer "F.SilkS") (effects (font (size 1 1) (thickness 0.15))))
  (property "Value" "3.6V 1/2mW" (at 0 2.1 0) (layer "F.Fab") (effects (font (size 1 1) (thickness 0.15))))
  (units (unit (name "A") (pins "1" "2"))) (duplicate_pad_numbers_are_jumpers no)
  (fp_line (start -2.36 -1) (end -2.36 1) (stroke (width 0.12) (type solid)) (layer "F.SilkS"))
  (fp_line (start -2.36 -1) (end 1.65 -1) (stroke (width 0.12) (type solid)) (layer "F.SilkS"))
  (fp_line (start -2.36 1) (end 1.65 1) (stroke (width 0.12) (type solid)) (layer "F.SilkS"))
  (pad "1" smd roundrect (at -1.65 0) (size 0.9 1.2) (layers "F.Cu" "F.Mask" "F.Paste") (roundrect_rratio 0.25) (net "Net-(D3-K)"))
  (pad "2" smd roundrect (at 1.65 0) (size 0.9 1.2) (layers "F.Cu" "F.Mask" "F.Paste") (roundrect_rratio 0.25) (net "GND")))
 (gr_line (start 141.5 95) (end 153.5 95) (stroke (width 0.1) (type default)) (layer "Edge.Cuts"))
 (gr_line (start 141.5 103.5) (end 141.5 95) (stroke (width 0.1) (type default)) (layer "Edge.Cuts"))
 (gr_line (start 141.5 123.5) (end 141.5 103.5) (stroke (width 0.1) (type default)) (layer "Edge.Cuts"))
 (gr_line (start 153.5 95) (end 153.5 103.5) (stroke (width 0.1) (type default)) (layer "Edge.Cuts"))
 (gr_line (start 153.5 103.5) (end 162.5 103.5) (stroke (width 0.1) (type default)) (layer "Edge.Cuts"))
 (gr_line (start 162.5 103.5) (end 172 103.5) (stroke (width 0.1) (type default)) (layer "Edge.Cuts"))
 (gr_line (start 172 103.5) (end 172 123.5) (stroke (width 0.1) (type default)) (layer "Edge.Cuts"))
 (gr_line (start 172 123.5) (end 141.5 123.5) (stroke (width 0.1) (type default)) (layer "Edge.Cuts"))
 (segment (start 145.96 120) (end 147.31 118.65) (width 0.6) (layer "F.Cu") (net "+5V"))
 (segment (start 155.2 116.3) (end 155.2 112.3) (width 0.6) (layer "F.Cu") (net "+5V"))
 (segment (start 152.85 118.65) (end 155.2 116.3) (width 0.6) (layer "F.Cu") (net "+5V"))
 (segment (start 161.4125 116.405) (end 162.224999 116.405) (width 0.6) (layer "F.Cu") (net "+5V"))
 (segment (start 147.825 110.2) (end 149.025 109) (width 0.6) (layer "F.Cu") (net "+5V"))
 (segment (start 143.5 109.25) (end 144.45 110.2) (width 0.6) (layer "F.Cu") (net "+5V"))
 (segment (start 162.725 111.725) (end 162.5 111.5) (width 0.6) (layer "F.Cu") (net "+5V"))
 (segment (start 144.45 110.2) (end 147.825 110.2) (width 0.6) (layer "F.Cu") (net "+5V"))
 (segment (start 155.2 112.3) (end 156 111.5) (width 0.6) (layer "F.Cu") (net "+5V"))
 (segment (start 154 109.5) (end 149.525 109.5) (width 0.6) (layer "F.Cu") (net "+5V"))
 (segment (start 162.5 111.5) (end 156 111.5) (width 0.6) (layer "F.Cu") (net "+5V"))
 (segment (start 147.31 118.65) (end 152.85 118.65) (width 0.6) (layer "F.Cu") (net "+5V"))
 (segment (start 156 111.5) (end 154 109.5) (width 0.6) (layer "F.Cu") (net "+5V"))
 (segment (start 145.55 116.6) (end 145.55 119.59) (width 0.6) (layer "F.Cu") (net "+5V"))
 (segment (start 145.55 119.59) (end 145.96 120) (width 0.6) (layer "F.Cu") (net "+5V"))
 (segment (start 162.224999 116.405) (end 162.725 115.904999) (width 0.6) (layer "F.Cu") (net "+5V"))
 (segment (start 149.525 109.5) (end 149.025 109) (width 0.6) (layer "F.Cu") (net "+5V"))
 (segment (start 162.725 115.904999) (end 162.725 111.725) (width 0.6) (layer "F.Cu") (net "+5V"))
 (segment (start 146.975 106.625) (end 146.85 106.5) (width 0.6) (layer "F.Cu") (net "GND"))
 (segment (start 144.482412 112.3) (end 144.45 112.332412) (width 0.6) (layer "F.Cu") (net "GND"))
 (segment (start 146.85 106.5) (end 145.25 108.1) (width 0.6) (layer "F.Cu") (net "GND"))
 (segment (start 151 99.8) (end 151 104) (width 0.6) (layer "F.Cu") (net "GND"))
 (segment (start 165.65 105.282412) (end 165.65 109) (width 0.6) (layer "F.Cu") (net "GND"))
 (segment (start 142.582412 108.1) (end 142.15 108.532412) (width 0.6) (layer "F.Cu") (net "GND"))
 (segment (start 142.15 108.532412) (end 142.15 109.967588) (width 0.6) (layer "F.Cu") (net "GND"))
 (segment (start 147 121.5) (end 148.5 120) (width 0.6) (layer "F.Cu") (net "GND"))
 (segment (start 165.65 112.15) (end 166.095 112.595) (width 0.6) (layer "F.Cu") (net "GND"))
 (segment (start 144.5 121.5) (end 147 121.5) (width 0.6) (layer "F.Cu") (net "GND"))
 (segment (start 145.25 108.1) (end 142.582412 108.1) (width 0.6) (layer "F.Cu") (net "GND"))
 (segment (start 151.5 104.5) (end 164.867588 104.5) (width 0.6) (layer "F.Cu") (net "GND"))
 (segment (start 150 115) (end 152 117) (width 0.6) (layer "F.Cu") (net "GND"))
 (segment (start 164.867588 104.5) (end 165.65 105.282412) (width 0.6) (layer "F.Cu") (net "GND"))
 (segment (start 144.45 112.332412) (end 144.45 121.45) (width 0.6) (layer "F.Cu") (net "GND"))
 (segment (start 166.095 112.595) (end 168.5875 112.595) (width 0.6) (layer "F.Cu") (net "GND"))
 (segment (start 144.482412 112.3) (end 148.3 112.3) (width 0.6) (layer "F.Cu") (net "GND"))
 (segment (start 142.15 109.967588) (end 144.482412 112.3) (width 0.6) (layer "F.Cu") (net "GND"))
 (segment (start 151 104) (end 151.5 104.5) (width 0.6) (layer "F.Cu") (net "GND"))
 (segment (start 148.3 112.3) (end 150 114) (width 0.6) (layer "F.Cu") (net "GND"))
 (segment (start 150 114) (end 150 115) (width 0.6) (layer "F.Cu") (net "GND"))
 (segment (start 146.975 109) (end 146.975 106.625) (width 0.6) (layer "F.Cu") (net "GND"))
 (segment (start 144.45 121.45) (end 144.5 121.5) (width 0.6) (layer "F.Cu") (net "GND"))
 (segment (start 165.65 109) (end 165.65 112.15) (width 0.6) (layer "F.Cu") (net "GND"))
 (segment (start 156 112.85) (end 156.255 112.595) (width 0.6) (layer "F.Cu") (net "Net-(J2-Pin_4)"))
 (segment (start 156.255 112.595) (end 161.4125 112.595) (width 0.6) (layer "F.Cu") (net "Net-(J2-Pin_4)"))
 (segment (start 153.58 120) (end 156 117.58) (width 0.6) (layer "F.Cu") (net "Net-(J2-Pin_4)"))
 (segment (start 156 117.58) (end 156 112.85) (width 0.6) (layer "F.Cu") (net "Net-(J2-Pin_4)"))
 (segment (start 157.1 119.02) (end 156.12 120) (width 0.6) (layer "F.Cu") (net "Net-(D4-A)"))
 (segment (start 157.1 113.95) (end 157.1 119.02) (width 0.6) (layer "F.Cu") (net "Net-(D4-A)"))
 (segment (start 161.4125 113.865) (end 157.185 113.865) (width 0.6) (layer "F.Cu") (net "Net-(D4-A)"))
 (segment (start 157.185 113.865) (end 157.1 113.95) (width 0.6) (layer "F.Cu") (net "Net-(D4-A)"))
 (segment (start 160.600001 115.135) (end 158.66 117.075001) (width 0.6) (layer "F.Cu") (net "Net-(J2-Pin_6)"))
 (segment (start 158.66 117.075001) (end 158.66 120) (width 0.6) (layer "F.Cu") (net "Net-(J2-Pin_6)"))
 (segment (start 161.4125 115.135) (end 160.600001 115.135) (width 0.6) (layer "F.Cu") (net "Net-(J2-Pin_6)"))
 (segment (start 166.372259 115.135) (end 166.065 115.135) (width 0.6) (layer "F.Cu") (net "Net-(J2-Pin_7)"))
 (segment (start 162.83137 110.7) (end 163.525 111.393629) (width 0.6) (layer "F.Cu") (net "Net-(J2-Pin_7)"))
 (segment (start 158 109.5) (end 159.2 110.7) (width 0.6) (layer "F.Cu") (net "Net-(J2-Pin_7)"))
 (segment (start 163.525 111.393629) (end 163.525 112.287741) (width 0.6) (layer "F.Cu") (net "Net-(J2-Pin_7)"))
 (segment (start 163.525 112.287741) (end 166.372259 115.135) (width 0.6) (layer "F.Cu") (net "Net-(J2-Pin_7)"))
 (segment (start 159.2 110.7) (end 162.83137 110.7) (width 0.6) (layer "F.Cu") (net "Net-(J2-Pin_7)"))
 (segment (start 166.065 115.135) (end 161.2 120) (width 0.6) (layer "F.Cu") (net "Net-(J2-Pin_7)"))
 (segment (start 166.372259 115.135) (end 168.5875 115.135) (width 0.6) (layer "F.Cu") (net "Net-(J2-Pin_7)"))
 (segment (start 164.5 112.13137) (end 166.23363 113.865) (width 0.6) (layer "F.Cu") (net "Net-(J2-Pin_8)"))
 (segment (start 164.5 106) (end 164.5 112.13137) (width 0.6) (layer "F.Cu") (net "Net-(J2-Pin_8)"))
 (segment (start 170.5 114.965001) (end 169.399999 113.865) (width 0.6) (layer "F.Cu") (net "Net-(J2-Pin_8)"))
 (segment (start 165.09 121.35) (end 169.379189 121.35) (width 0.6) (layer "F.Cu") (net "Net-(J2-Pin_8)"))
 (segment (start 169.379189 121.35) (end 170.5 120.229189) (width 0.6) (layer "F.Cu") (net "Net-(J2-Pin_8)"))
 (segment (start 170.5 120.229189) (end 170.5 114.965001) (width 0.6) (layer "F.Cu") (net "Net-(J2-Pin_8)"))
 (segment (start 166.23363 113.865) (end 168.5875 113.865) (width 0.6) (layer "F.Cu") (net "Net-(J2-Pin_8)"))
 (segment (start 169.399999 113.865) (end 168.5875 113.865) (width 0.6) (layer "F.Cu") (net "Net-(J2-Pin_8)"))
 (segment (start 163.74 120) (end 165.09 121.35) (width 0.6) (layer "F.Cu") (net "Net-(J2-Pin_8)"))
 (segment (start 166.28 120) (end 166.28 118.7125) (width 0.6) (layer "F.Cu") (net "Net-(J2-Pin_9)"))
 (segment (start 166.28 118.7125) (end 168.5875 116.405) (width 0.6) (layer "F.Cu") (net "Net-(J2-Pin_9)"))
 (segment (start 144 99.8) (end 144 105.25) (width 0.6) (layer "F.Cu") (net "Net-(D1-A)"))
 (segment (start 144 105.25) (end 143.5 105.75) (width 0.6) (layer "F.Cu") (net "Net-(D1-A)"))
 (segment (start 151 106.5) (end 152 107.5) (width 0.6) (layer "F.Cu") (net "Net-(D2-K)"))
 (segment (start 152 107.5) (end 154 107.5) (width 0.6) (layer "F.Cu") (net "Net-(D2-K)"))
 (segment (start 149.05 105.4) (end 150.15 106.5) (width 0.6) (layer "F.Cu") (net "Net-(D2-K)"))
 (segment (start 146.5 104.9) (end 147 105.4) (width 0.6) (layer "F.Cu") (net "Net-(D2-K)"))
 (segment (start 150.15 106.5) (end 151 106.5) (width 0.6) (layer "F.Cu") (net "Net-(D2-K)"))
 (segment (start 146.5 100.3) (end 146.5 104.9) (width 0.6) (layer "F.Cu") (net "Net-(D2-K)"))
 (segment (start 154 107.5) (end 158 107.5) (width 0.6) (layer "F.Cu") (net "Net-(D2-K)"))
 (segment (start 147 105.4) (end 149.05 105.4) (width 0.6) (layer "F.Cu") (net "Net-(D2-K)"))
 (segment (start 151.131371 105.5) (end 151.63137 106) (width 0.6) (layer "F.Cu") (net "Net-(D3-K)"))
 (segment (start 162.35 109) (end 162.35 106.15) (width 0.6) (layer "F.Cu") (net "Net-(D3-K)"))
 (segment (start 150 104.5) (end 151 105.5) (width 0.6) (layer "F.Cu") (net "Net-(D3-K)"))
 (segment (start 162.35 106.15) (end 162.5 106) (width 0.6) (layer "F.Cu") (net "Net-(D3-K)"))
 (segment (start 151 105.5) (end 151.131371 105.5) (width 0.6) (layer "F.Cu") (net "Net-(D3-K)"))
 (segment (start 151.63137 106) (end 162.5 106) (width 0.6) (layer "F.Cu") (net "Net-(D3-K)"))
 (segment (start 148.5 104.5) (end 150 104.5) (width 0.6) (layer "F.Cu") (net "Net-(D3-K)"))
 (segment (start 148.5 100.3) (end 148.5 104.5) (width 0.6) (layer "F.Cu") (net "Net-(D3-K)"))
 (segment (start 146.4 113.4) (end 150 117) (width 0.6) (layer "F.Cu") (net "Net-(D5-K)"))
 (segment (start 145.55 113.4) (end 146.4 113.4) (width 0.6) (layer "F.Cu") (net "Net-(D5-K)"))
 (segment (start 151.95 113.95) (end 150 112) (width 0.6) (layer "F.Cu") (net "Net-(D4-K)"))
 (segment (start 153.9 113.95) (end 151.95 113.95) (width 0.6) (layer "F.Cu") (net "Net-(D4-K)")))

